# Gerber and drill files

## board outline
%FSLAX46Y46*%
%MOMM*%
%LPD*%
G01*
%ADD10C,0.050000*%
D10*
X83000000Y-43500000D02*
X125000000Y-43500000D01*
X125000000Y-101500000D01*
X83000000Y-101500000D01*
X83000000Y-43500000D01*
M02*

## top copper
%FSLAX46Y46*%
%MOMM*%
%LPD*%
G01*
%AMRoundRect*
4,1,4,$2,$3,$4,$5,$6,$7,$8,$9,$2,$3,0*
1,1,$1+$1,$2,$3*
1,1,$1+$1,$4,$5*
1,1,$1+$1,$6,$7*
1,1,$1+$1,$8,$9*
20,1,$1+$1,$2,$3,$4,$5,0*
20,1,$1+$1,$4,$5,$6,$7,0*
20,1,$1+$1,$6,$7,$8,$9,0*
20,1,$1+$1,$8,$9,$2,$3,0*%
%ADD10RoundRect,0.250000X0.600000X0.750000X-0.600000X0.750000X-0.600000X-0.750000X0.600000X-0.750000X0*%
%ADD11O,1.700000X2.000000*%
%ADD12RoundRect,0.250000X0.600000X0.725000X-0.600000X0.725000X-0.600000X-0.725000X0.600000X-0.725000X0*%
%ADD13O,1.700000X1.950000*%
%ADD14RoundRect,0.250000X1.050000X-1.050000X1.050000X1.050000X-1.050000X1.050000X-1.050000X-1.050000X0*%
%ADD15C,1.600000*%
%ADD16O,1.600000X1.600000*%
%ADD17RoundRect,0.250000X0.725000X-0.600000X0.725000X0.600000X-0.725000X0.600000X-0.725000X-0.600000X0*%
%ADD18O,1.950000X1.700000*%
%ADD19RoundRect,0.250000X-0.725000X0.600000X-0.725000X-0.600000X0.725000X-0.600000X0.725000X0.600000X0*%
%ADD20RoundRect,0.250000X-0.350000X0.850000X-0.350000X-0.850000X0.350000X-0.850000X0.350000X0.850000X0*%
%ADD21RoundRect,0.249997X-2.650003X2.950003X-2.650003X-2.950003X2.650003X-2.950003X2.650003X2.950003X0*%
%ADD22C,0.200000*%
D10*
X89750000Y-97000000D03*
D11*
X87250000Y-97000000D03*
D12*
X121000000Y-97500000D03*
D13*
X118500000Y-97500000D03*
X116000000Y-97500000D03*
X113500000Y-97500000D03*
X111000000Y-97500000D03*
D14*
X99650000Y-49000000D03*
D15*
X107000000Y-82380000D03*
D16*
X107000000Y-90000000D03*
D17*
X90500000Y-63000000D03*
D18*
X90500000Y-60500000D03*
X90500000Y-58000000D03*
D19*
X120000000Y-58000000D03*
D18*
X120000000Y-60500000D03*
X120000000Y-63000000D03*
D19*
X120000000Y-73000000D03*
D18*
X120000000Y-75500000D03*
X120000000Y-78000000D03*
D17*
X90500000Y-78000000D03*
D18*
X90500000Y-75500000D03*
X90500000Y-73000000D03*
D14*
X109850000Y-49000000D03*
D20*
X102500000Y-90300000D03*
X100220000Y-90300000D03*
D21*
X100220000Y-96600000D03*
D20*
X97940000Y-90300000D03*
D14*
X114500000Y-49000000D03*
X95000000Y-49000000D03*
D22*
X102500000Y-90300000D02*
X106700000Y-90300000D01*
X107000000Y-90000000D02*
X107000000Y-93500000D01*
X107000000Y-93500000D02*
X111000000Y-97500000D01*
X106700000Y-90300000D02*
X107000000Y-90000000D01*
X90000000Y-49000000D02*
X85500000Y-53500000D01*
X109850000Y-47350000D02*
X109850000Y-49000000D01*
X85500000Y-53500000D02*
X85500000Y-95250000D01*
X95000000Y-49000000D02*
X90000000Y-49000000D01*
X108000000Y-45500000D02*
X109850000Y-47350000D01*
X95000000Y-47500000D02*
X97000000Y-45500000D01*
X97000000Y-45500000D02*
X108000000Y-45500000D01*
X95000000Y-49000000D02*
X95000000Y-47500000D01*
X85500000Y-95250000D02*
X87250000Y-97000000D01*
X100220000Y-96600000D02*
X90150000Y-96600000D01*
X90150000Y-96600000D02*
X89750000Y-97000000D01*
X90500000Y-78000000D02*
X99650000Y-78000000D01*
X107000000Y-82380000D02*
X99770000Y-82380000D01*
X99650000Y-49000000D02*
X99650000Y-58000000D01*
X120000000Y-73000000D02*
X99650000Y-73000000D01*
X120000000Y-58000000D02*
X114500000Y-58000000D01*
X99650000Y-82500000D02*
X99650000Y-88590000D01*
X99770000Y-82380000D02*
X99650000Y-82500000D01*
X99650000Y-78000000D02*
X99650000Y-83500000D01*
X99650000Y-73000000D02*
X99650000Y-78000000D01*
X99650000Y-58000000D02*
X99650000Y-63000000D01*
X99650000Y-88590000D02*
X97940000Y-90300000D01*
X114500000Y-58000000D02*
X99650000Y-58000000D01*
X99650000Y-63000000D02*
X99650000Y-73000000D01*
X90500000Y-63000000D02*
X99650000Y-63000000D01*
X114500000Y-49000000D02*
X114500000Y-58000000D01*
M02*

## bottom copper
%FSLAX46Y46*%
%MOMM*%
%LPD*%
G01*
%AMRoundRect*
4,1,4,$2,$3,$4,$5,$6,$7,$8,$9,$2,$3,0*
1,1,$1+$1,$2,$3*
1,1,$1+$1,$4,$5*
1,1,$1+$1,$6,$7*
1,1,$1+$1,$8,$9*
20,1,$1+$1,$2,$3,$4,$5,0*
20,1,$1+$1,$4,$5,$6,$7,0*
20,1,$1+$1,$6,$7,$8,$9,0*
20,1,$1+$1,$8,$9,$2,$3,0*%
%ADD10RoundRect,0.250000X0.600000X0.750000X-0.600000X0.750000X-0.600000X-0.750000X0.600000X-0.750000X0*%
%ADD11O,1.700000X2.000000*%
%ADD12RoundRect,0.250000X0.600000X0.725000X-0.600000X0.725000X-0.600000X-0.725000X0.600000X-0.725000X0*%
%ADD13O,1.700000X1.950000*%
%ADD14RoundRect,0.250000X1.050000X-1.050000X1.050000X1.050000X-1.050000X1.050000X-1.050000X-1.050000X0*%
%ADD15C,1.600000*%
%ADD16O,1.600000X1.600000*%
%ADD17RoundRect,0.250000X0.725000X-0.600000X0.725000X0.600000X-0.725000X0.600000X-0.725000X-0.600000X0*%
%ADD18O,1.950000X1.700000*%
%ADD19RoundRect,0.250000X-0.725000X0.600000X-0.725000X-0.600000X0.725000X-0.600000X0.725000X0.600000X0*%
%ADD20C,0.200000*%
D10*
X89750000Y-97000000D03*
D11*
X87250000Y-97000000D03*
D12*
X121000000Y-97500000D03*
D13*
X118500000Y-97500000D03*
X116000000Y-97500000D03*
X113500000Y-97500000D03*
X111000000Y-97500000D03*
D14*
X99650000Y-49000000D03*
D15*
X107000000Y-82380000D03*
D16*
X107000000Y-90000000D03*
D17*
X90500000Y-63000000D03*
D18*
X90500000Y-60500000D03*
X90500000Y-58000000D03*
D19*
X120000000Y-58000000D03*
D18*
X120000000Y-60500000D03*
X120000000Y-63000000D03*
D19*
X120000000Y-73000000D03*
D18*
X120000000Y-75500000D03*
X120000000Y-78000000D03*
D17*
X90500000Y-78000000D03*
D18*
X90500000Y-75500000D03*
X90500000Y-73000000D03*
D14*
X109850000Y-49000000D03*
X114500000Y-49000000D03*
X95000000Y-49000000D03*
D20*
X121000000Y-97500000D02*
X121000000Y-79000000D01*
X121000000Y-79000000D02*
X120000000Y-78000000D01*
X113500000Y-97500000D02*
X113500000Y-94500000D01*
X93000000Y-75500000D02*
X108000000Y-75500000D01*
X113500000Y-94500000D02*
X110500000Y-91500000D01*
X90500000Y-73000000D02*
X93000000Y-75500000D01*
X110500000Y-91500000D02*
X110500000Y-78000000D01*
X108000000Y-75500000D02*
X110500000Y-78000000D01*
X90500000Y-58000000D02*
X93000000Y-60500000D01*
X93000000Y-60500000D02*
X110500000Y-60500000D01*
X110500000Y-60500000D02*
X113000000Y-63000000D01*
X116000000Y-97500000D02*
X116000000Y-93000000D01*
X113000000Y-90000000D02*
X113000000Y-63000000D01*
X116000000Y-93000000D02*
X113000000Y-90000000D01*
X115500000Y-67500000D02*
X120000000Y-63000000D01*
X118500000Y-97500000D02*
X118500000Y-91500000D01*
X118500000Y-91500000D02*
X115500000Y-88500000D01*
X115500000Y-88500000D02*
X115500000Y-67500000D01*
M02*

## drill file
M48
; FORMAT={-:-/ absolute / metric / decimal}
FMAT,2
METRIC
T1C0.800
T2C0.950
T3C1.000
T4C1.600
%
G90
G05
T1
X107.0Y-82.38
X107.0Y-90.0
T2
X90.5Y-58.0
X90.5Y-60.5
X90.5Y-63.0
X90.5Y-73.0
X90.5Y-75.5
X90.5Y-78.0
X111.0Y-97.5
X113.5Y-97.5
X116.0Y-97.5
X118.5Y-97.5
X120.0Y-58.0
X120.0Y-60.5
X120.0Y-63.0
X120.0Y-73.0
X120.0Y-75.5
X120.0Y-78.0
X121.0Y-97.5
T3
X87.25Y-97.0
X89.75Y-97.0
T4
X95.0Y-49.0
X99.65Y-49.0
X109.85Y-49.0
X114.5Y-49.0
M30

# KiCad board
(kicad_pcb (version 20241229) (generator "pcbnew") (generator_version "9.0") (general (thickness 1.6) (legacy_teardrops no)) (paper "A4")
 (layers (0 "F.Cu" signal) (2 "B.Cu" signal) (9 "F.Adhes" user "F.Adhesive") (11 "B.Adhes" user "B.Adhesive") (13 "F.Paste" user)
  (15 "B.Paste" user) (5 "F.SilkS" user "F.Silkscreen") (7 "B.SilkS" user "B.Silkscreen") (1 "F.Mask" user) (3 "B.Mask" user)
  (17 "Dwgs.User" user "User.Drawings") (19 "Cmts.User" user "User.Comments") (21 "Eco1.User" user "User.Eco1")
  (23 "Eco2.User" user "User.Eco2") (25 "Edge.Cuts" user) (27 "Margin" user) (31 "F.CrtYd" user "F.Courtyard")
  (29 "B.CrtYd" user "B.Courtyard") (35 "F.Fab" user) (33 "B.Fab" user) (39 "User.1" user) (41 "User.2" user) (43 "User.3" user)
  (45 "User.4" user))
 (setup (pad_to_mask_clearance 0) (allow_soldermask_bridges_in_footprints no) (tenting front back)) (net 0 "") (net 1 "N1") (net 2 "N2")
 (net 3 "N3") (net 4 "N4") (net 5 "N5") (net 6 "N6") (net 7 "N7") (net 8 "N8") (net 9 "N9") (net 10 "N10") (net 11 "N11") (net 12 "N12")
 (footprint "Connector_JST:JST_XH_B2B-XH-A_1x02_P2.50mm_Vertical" (layer "F.Cu") (at 89.75 97 180)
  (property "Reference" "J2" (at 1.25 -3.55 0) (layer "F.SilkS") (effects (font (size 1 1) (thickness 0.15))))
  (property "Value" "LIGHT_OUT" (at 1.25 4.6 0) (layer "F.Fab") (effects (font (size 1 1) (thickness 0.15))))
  (pad "1" thru_hole roundrect (at 0 0 180) (size 1.7 2) (drill 1) (layers "*.Cu" "*.Mask") (remove_unused_layers no)
   (roundrect_rratio 0.147059) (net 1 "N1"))
  (pad "2" thru_hole oval (at 2.5 0 180) (size 1.7 2) (drill 1) (layers "*.Cu" "*.Mask") (remove_unused_layers no) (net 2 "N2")))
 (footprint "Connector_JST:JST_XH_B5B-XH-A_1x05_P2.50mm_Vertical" (layer "F.Cu") (at 121 97.5 180)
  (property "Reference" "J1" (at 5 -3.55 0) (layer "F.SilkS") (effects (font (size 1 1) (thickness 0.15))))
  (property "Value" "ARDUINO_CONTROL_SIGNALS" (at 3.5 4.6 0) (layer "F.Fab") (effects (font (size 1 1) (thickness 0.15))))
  (pad "1" thru_hole roundrect (at 0 0 180) (size 1.7 1.95) (drill 0.95) (layers "*.Cu" "*.Mask") (remove_unused_layers no)
   (roundrect_rratio 0.147059) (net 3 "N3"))
  (pad "2" thru_hole oval (at 2.5 0 180) (size 1.7 1.95) (drill 0.95) (layers "*.Cu" "*.Mask") (remove_unused_layers no) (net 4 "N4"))
  (pad "3" thru_hole oval (at 5 0 180) (size 1.7 1.95) (drill 0.95) (layers "*.Cu" "*.Mask") (remove_unused_layers no) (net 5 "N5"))
  (pad "4" thru_hole oval (at 7.5 0 180) (size 1.7 1.95) (drill 0.95) (layers "*.Cu" "*.Mask") (remove_unused_layers no) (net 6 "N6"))
  (pad "5" thru_hole oval (at 10 0 180) (size 1.7 1.95) (drill 0.95) (layers "*.Cu" "*.Mask") (remove_unused_layers no) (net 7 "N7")))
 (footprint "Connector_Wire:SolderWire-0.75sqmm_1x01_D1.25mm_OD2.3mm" (layer "F.Cu") (at 99.65 49 90)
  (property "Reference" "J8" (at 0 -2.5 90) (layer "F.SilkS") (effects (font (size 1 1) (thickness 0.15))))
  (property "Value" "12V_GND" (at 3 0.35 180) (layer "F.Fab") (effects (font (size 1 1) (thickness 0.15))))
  (pad "1" thru_hole roundrect (at 0 0 90) (size 2.6 2.6) (drill 1.6) (layers "*.Cu" "*.Mask") (remove_unused_layers no)
   (roundrect_rratio 0.096154) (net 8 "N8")))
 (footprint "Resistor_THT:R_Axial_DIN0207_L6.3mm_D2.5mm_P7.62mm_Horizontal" (layer "F.Cu") (at 107 82.38 -90)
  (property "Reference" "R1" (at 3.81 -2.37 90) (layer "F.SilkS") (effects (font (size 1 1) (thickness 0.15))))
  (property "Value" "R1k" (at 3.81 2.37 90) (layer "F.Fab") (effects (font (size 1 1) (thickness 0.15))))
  (pad "1" thru_hole circle (at 0 0 270) (size 1.6 1.6) (drill 0.8) (layers "*.Cu" "*.Mask") (remove_unused_layers no) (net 8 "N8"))
  (pad "2" thru_hole oval (at 7.62 0 270) (size 1.6 1.6) (drill 0.8) (layers "*.Cu" "*.Mask") (remove_unused_layers no) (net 7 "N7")))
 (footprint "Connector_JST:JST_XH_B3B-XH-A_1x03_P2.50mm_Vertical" (layer "F.Cu") (at 90.5 63 90)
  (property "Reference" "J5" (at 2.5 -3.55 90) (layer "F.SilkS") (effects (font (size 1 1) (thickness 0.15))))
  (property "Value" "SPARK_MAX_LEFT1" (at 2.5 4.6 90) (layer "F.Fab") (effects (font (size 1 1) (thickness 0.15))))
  (pad "1" thru_hole roundrect (at 0 0 90) (size 1.7 1.95) (drill 0.95) (layers "*.Cu" "*.Mask") (remove_unused_layers no)
   (roundrect_rratio 0.147059) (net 8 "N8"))
  (pad "2" thru_hole oval (at 2.5 0 90) (size 1.7 1.95) (drill 0.95) (layers "*.Cu" "*.Mask") (remove_unused_layers no) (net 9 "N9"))
  (pad "3" thru_hole oval (at 5 0 90) (size 1.7 1.95) (drill 0.95) (layers "*.Cu" "*.Mask") (remove_unused_layers no) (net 5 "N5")))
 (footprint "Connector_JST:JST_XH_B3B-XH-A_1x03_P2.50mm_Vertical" (layer "F.Cu") (at 120 58 -90)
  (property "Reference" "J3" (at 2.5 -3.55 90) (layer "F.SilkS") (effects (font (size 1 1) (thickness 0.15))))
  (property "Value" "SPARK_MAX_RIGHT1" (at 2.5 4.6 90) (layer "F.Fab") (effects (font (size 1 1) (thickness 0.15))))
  (pad "1" thru_hole roundrect (at 0 0 270) (size 1.7 1.95) (drill 0.95) (layers "*.Cu" "*.Mask") (remove_unused_layers no)
   (roundrect_rratio 0.147059) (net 8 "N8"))
  (pad "2" thru_hole oval (at 2.5 0 270) (size 1.7 1.95) (drill 0.95) (layers "*.Cu" "*.Mask") (remove_unused_layers no) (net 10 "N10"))
  (pad "3" thru_hole oval (at 5 0 270) (size 1.7 1.95) (drill 0.95) (layers "*.Cu" "*.Mask") (remove_unused_layers no) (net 4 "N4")))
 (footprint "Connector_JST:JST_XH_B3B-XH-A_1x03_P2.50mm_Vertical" (layer "F.Cu") (at 120 73 -90)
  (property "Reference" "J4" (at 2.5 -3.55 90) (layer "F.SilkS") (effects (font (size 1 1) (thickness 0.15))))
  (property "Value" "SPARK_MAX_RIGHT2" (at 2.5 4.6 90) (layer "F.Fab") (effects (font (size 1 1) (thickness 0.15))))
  (pad "1" thru_hole roundrect (at 0 0 270) (size 1.7 1.95) (drill 0.95) (layers "*.Cu" "*.Mask") (remove_unused_layers no)
   (roundrect_rratio 0.147059) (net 8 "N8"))
  (pad "2" thru_hole oval (at 2.5 0 270) (size 1.7 1.95) (drill 0.95) (layers "*.Cu" "*.Mask") (remove_unused_layers no) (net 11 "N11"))
  (pad "3" thru_hole oval (at 5 0 270) (size 1.7 1.95) (drill 0.95) (layers "*.Cu" "*.Mask") (remove_unused_layers no) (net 3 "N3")))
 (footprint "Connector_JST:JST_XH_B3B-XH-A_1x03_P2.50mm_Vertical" (layer "F.Cu") (at 90.5 78 90)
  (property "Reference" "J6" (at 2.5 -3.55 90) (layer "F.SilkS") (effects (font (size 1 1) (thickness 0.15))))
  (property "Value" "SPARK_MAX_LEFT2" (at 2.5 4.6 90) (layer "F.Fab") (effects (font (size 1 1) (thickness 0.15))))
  (pad "1" thru_hole roundrect (at 0 0 90) (size 1.7 1.95) (drill 0.95) (layers "*.Cu" "*.Mask") (remove_unused_layers no)
   (roundrect_rratio 0.147059) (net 8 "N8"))
  (pad "2" thru_hole oval (at 2.5 0 90) (size 1.7 1.95) (drill 0.95) (layers "*.Cu" "*.Mask") (remove_unused_layers no) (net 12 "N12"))
  (pad "3" thru_hole oval (at 5 0 90) (size 1.7 1.95) (drill 0.95) (layers "*.Cu" "*.Mask") (remove_unused_layers no) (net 6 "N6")))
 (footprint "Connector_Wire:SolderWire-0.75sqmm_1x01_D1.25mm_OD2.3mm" (layer "F.Cu") (at 109.85 49 90)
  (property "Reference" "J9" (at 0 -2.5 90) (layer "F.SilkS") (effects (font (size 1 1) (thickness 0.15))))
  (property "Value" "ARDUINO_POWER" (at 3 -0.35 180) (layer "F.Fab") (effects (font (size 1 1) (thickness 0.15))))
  (pad "1" thru_hole roundrect (at 0 0 90) (size 2.6 2.6) (drill 1.6) (layers "*.Cu" "*.Mask") (remove_unused_layers no)
   (roundrect_rratio 0.096154) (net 2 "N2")))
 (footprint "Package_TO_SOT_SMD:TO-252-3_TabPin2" (layer "F.Cu") (at 100.22 95.34 -90)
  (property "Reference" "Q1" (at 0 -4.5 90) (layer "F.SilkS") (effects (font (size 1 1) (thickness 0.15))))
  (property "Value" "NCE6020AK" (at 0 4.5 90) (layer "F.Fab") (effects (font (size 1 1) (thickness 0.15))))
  (pad "" smd roundrect (at -0.415 -1.525 270) (size 3.05 2.75) (layers "F.Paste") (roundrect_rratio 0.090909))
  (pad "" smd roundrect (at -0.415 1.525 270) (size 3.05 2.75) (layers "F.Paste") (roundrect_rratio 0.090909))
  (pad "" smd roundrect (at 2.935 -1.525 270) (size 3.05 2.75) (layers "F.Paste") (roundrect_rratio 0.090909))
  (pad "" smd roundrect (at 2.935 1.525 270) (size 3.05 2.75) (layers "F.Paste") (roundrect_rratio 0.090909))
  (pad "1" smd roundrect (at -5.04 -2.28 270) (size 2.2 1.2) (layers "F.Cu" "F.Mask" "F.Paste") (roundrect_rratio 0.208333) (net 7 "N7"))
  (pad "2" smd roundrect (at -5.04 0 270) (size 2.2 1.2) (layers "F.Cu" "F.Mask" "F.Paste") (roundrect_rratio 0.208333) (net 1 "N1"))
  (pad "2" smd roundrect (at 1.26 0 270) (size 6.4 5.8) (layers "F.Cu" "F.Mask") (roundrect_rratio 0.043103) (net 1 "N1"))
  (pad "3" smd roundrect (at -5.04 2.28 270) (size 2.2 1.2) (layers "F.Cu" "F.Mask" "F.Paste") (roundrect_rratio 0.208333) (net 8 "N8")))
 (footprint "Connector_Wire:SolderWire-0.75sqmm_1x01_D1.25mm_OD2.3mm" (layer "F.Cu") (at 114.5 49 90)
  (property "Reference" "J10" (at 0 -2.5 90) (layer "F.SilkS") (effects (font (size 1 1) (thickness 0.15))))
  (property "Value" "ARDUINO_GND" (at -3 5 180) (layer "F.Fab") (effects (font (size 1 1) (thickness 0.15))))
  (pad "1" thru_hole roundrect (at 0 0 90) (size 2.6 2.6) (drill 1.6) (layers "*.Cu" "*.Mask") (remove_unused_layers no)
   (roundrect_rratio 0.096154) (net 8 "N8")))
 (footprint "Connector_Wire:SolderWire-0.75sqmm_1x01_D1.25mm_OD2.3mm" (layer "F.Cu") (at 95 49 90)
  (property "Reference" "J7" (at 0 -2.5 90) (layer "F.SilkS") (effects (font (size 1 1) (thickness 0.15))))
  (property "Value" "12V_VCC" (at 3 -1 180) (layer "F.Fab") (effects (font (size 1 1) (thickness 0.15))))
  (pad "1" thru_hole roundrect (at 0 0 90) (size 2.6 2.6) (drill 1.6) (layers "*.Cu" "*.Mask") (remove_unused_layers no)
   (roundrect_rratio 0.096154) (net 2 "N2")))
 (gr_rect (start 83 43.5) (end 125 101.5) (stroke (width 0.05) (type default)) (fill no) (layer "Edge.Cuts"))
 (segment (start 121 97.5) (end 121 79) (width 0.2) (layer "B.Cu") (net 3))
 (segment (start 121 79) (end 120 78) (width 0.2) (layer "B.Cu") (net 3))
 (segment (start 113.5 97.5) (end 113.5 94.5) (width 0.2) (layer "B.Cu") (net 6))
 (segment (start 93 75.5) (end 108 75.5) (width 0.2) (layer "B.Cu") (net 6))
 (segment (start 113.5 94.5) (end 110.5 91.5) (width 0.2) (layer "B.Cu") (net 6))
 (segment (start 90.5 73) (end 93 75.5) (width 0.2) (layer "B.Cu") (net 6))
 (segment (start 110.5 91.5) (end 110.5 78) (width 0.2) (layer "B.Cu") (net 6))
 (segment (start 108 75.5) (end 110.5 78) (width 0.2) (layer "B.Cu") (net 6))
 (segment (start 90.5 58) (end 93 60.5) (width 0.2) (layer "B.Cu") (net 5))
 (segment (start 93 60.5) (end 110.5 60.5) (width 0.2) (layer "B.Cu") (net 5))
 (segment (start 110.5 60.5) (end 113 63) (width 0.2) (layer "B.Cu") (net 5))
 (segment (start 116 97.5) (end 116 93) (width 0.2) (layer "B.Cu") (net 5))
 (segment (start 113 90) (end 113 63) (width 0.2) (layer "B.Cu") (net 5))
 (segment (start 116 93) (end 113 90) (width 0.2) (layer "B.Cu") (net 5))
 (segment (start 102.5 90.3) (end 106.7 90.3) (width 0.2) (layer "F.Cu") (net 7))
 (segment (start 107 90) (end 107 93.5) (width 0.2) (layer "F.Cu") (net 7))
 (segment (start 107 93.5) (end 111 97.5) (width 0.2) (layer "F.Cu") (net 7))
 (segment (start 106.7 90.3) (end 107 90) (width 0.2) (layer "F.Cu") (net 7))
 (segment (start 115.5 67.5) (end 120 63) (width 0.2) (layer "B.Cu") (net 4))
 (segment (start 118.5 97.5) (end 118.5 91.5) (width 0.2) (layer "B.Cu") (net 4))
 (segment (start 118.5 91.5) (end 115.5 88.5) (width 0.2) (layer "B.Cu") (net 4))
 (segment (start 115.5 88.5) (end 115.5 67.5) (width 0.2) (layer "B.Cu") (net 4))
 (segment (start 90 49) (end 85.5 53.5) (width 0.2) (layer "F.Cu") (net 2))
 (segment (start 109.85 47.35) (end 109.85 49) (width 0.2) (layer "F.Cu") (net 2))
 (segment (start 85.5 53.5) (end 85.5 95.25) (width 0.2) (layer "F.Cu") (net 2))
 (segment (start 95 49) (end 90 49) (width 0.2) (layer "F.Cu") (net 2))
 (segment (start 108 45.5) (end 109.85 47.35) (width 0.2) (layer "F.Cu") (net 2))
 (segment (start 95 47.5) (end 97 45.5) (width 0.2) (layer "F.Cu") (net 2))
 (segment (start 97 45.5) (end 108 45.5) (width 0.2) (layer "F.Cu") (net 2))
 (segment (start 95 49) (end 95 47.5) (width 0.2) (layer "F.Cu") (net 2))
 (segment (start 85.5 95.25) (end 87.25 97) (width 0.2) (layer "F.Cu") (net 2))
 (segment (start 100.22 96.6) (end 90.15 96.6) (width 0.2) (layer "F.Cu") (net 1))
 (segment (start 90.15 96.6) (end 89.75 97) (width 0.2) (layer "F.Cu") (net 1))
 (segment (start 90.5 78) (end 99.65 78) (width 0.2) (layer "F.Cu") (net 8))
 (segment (start 107 82.38) (end 99.77 82.38) (width 0.2) (layer "F.Cu") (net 8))
 (segment (start 99.65 49) (end 99.65 58) (width 0.2) (layer "F.Cu") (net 8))
 (segment (start 120 73) (end 99.65 73) (width 0.2) (layer "F.Cu") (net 8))
 (segment (start 120 58) (end 114.5 58) (width 0.2) (layer "F.Cu") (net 8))
 (segment (start 99.65 82.5) (end 99.65 88.59) (width 0.2) (layer "F.Cu") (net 8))
 (segment (start 99.77 82.38) (end 99.65 82.5) (width 0.2) (layer "F.Cu") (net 8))
 (segment (start 99.65 78) (end 99.65 83.5) (width 0.2) (layer "F.Cu") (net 8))
 (segment (start 99.65 73) (end 99.65 78) (width 0.2) (layer "F.Cu") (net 8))
 (segment (start 99.65 58) (end 99.65 63) (width 0.2) (layer "F.Cu") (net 8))
 (segment (start 99.65 88.59) (end 97.94 90.3) (width 0.2) (layer "F.Cu") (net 8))
 (segment (start 114.5 58) (end 99.65 58) (width 0.2) (layer "F.Cu") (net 8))
 (segment (start 99.65 63) (end 99.65 73) (width 0.2) (layer "F.Cu") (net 8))
 (segment (start 90.5 63) (end 99.65 63) (width 0.2) (layer "F.Cu") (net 8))
 (segment (start 114.5 49) (end 114.5 58) (width 0.2) (layer "F.Cu") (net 8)))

